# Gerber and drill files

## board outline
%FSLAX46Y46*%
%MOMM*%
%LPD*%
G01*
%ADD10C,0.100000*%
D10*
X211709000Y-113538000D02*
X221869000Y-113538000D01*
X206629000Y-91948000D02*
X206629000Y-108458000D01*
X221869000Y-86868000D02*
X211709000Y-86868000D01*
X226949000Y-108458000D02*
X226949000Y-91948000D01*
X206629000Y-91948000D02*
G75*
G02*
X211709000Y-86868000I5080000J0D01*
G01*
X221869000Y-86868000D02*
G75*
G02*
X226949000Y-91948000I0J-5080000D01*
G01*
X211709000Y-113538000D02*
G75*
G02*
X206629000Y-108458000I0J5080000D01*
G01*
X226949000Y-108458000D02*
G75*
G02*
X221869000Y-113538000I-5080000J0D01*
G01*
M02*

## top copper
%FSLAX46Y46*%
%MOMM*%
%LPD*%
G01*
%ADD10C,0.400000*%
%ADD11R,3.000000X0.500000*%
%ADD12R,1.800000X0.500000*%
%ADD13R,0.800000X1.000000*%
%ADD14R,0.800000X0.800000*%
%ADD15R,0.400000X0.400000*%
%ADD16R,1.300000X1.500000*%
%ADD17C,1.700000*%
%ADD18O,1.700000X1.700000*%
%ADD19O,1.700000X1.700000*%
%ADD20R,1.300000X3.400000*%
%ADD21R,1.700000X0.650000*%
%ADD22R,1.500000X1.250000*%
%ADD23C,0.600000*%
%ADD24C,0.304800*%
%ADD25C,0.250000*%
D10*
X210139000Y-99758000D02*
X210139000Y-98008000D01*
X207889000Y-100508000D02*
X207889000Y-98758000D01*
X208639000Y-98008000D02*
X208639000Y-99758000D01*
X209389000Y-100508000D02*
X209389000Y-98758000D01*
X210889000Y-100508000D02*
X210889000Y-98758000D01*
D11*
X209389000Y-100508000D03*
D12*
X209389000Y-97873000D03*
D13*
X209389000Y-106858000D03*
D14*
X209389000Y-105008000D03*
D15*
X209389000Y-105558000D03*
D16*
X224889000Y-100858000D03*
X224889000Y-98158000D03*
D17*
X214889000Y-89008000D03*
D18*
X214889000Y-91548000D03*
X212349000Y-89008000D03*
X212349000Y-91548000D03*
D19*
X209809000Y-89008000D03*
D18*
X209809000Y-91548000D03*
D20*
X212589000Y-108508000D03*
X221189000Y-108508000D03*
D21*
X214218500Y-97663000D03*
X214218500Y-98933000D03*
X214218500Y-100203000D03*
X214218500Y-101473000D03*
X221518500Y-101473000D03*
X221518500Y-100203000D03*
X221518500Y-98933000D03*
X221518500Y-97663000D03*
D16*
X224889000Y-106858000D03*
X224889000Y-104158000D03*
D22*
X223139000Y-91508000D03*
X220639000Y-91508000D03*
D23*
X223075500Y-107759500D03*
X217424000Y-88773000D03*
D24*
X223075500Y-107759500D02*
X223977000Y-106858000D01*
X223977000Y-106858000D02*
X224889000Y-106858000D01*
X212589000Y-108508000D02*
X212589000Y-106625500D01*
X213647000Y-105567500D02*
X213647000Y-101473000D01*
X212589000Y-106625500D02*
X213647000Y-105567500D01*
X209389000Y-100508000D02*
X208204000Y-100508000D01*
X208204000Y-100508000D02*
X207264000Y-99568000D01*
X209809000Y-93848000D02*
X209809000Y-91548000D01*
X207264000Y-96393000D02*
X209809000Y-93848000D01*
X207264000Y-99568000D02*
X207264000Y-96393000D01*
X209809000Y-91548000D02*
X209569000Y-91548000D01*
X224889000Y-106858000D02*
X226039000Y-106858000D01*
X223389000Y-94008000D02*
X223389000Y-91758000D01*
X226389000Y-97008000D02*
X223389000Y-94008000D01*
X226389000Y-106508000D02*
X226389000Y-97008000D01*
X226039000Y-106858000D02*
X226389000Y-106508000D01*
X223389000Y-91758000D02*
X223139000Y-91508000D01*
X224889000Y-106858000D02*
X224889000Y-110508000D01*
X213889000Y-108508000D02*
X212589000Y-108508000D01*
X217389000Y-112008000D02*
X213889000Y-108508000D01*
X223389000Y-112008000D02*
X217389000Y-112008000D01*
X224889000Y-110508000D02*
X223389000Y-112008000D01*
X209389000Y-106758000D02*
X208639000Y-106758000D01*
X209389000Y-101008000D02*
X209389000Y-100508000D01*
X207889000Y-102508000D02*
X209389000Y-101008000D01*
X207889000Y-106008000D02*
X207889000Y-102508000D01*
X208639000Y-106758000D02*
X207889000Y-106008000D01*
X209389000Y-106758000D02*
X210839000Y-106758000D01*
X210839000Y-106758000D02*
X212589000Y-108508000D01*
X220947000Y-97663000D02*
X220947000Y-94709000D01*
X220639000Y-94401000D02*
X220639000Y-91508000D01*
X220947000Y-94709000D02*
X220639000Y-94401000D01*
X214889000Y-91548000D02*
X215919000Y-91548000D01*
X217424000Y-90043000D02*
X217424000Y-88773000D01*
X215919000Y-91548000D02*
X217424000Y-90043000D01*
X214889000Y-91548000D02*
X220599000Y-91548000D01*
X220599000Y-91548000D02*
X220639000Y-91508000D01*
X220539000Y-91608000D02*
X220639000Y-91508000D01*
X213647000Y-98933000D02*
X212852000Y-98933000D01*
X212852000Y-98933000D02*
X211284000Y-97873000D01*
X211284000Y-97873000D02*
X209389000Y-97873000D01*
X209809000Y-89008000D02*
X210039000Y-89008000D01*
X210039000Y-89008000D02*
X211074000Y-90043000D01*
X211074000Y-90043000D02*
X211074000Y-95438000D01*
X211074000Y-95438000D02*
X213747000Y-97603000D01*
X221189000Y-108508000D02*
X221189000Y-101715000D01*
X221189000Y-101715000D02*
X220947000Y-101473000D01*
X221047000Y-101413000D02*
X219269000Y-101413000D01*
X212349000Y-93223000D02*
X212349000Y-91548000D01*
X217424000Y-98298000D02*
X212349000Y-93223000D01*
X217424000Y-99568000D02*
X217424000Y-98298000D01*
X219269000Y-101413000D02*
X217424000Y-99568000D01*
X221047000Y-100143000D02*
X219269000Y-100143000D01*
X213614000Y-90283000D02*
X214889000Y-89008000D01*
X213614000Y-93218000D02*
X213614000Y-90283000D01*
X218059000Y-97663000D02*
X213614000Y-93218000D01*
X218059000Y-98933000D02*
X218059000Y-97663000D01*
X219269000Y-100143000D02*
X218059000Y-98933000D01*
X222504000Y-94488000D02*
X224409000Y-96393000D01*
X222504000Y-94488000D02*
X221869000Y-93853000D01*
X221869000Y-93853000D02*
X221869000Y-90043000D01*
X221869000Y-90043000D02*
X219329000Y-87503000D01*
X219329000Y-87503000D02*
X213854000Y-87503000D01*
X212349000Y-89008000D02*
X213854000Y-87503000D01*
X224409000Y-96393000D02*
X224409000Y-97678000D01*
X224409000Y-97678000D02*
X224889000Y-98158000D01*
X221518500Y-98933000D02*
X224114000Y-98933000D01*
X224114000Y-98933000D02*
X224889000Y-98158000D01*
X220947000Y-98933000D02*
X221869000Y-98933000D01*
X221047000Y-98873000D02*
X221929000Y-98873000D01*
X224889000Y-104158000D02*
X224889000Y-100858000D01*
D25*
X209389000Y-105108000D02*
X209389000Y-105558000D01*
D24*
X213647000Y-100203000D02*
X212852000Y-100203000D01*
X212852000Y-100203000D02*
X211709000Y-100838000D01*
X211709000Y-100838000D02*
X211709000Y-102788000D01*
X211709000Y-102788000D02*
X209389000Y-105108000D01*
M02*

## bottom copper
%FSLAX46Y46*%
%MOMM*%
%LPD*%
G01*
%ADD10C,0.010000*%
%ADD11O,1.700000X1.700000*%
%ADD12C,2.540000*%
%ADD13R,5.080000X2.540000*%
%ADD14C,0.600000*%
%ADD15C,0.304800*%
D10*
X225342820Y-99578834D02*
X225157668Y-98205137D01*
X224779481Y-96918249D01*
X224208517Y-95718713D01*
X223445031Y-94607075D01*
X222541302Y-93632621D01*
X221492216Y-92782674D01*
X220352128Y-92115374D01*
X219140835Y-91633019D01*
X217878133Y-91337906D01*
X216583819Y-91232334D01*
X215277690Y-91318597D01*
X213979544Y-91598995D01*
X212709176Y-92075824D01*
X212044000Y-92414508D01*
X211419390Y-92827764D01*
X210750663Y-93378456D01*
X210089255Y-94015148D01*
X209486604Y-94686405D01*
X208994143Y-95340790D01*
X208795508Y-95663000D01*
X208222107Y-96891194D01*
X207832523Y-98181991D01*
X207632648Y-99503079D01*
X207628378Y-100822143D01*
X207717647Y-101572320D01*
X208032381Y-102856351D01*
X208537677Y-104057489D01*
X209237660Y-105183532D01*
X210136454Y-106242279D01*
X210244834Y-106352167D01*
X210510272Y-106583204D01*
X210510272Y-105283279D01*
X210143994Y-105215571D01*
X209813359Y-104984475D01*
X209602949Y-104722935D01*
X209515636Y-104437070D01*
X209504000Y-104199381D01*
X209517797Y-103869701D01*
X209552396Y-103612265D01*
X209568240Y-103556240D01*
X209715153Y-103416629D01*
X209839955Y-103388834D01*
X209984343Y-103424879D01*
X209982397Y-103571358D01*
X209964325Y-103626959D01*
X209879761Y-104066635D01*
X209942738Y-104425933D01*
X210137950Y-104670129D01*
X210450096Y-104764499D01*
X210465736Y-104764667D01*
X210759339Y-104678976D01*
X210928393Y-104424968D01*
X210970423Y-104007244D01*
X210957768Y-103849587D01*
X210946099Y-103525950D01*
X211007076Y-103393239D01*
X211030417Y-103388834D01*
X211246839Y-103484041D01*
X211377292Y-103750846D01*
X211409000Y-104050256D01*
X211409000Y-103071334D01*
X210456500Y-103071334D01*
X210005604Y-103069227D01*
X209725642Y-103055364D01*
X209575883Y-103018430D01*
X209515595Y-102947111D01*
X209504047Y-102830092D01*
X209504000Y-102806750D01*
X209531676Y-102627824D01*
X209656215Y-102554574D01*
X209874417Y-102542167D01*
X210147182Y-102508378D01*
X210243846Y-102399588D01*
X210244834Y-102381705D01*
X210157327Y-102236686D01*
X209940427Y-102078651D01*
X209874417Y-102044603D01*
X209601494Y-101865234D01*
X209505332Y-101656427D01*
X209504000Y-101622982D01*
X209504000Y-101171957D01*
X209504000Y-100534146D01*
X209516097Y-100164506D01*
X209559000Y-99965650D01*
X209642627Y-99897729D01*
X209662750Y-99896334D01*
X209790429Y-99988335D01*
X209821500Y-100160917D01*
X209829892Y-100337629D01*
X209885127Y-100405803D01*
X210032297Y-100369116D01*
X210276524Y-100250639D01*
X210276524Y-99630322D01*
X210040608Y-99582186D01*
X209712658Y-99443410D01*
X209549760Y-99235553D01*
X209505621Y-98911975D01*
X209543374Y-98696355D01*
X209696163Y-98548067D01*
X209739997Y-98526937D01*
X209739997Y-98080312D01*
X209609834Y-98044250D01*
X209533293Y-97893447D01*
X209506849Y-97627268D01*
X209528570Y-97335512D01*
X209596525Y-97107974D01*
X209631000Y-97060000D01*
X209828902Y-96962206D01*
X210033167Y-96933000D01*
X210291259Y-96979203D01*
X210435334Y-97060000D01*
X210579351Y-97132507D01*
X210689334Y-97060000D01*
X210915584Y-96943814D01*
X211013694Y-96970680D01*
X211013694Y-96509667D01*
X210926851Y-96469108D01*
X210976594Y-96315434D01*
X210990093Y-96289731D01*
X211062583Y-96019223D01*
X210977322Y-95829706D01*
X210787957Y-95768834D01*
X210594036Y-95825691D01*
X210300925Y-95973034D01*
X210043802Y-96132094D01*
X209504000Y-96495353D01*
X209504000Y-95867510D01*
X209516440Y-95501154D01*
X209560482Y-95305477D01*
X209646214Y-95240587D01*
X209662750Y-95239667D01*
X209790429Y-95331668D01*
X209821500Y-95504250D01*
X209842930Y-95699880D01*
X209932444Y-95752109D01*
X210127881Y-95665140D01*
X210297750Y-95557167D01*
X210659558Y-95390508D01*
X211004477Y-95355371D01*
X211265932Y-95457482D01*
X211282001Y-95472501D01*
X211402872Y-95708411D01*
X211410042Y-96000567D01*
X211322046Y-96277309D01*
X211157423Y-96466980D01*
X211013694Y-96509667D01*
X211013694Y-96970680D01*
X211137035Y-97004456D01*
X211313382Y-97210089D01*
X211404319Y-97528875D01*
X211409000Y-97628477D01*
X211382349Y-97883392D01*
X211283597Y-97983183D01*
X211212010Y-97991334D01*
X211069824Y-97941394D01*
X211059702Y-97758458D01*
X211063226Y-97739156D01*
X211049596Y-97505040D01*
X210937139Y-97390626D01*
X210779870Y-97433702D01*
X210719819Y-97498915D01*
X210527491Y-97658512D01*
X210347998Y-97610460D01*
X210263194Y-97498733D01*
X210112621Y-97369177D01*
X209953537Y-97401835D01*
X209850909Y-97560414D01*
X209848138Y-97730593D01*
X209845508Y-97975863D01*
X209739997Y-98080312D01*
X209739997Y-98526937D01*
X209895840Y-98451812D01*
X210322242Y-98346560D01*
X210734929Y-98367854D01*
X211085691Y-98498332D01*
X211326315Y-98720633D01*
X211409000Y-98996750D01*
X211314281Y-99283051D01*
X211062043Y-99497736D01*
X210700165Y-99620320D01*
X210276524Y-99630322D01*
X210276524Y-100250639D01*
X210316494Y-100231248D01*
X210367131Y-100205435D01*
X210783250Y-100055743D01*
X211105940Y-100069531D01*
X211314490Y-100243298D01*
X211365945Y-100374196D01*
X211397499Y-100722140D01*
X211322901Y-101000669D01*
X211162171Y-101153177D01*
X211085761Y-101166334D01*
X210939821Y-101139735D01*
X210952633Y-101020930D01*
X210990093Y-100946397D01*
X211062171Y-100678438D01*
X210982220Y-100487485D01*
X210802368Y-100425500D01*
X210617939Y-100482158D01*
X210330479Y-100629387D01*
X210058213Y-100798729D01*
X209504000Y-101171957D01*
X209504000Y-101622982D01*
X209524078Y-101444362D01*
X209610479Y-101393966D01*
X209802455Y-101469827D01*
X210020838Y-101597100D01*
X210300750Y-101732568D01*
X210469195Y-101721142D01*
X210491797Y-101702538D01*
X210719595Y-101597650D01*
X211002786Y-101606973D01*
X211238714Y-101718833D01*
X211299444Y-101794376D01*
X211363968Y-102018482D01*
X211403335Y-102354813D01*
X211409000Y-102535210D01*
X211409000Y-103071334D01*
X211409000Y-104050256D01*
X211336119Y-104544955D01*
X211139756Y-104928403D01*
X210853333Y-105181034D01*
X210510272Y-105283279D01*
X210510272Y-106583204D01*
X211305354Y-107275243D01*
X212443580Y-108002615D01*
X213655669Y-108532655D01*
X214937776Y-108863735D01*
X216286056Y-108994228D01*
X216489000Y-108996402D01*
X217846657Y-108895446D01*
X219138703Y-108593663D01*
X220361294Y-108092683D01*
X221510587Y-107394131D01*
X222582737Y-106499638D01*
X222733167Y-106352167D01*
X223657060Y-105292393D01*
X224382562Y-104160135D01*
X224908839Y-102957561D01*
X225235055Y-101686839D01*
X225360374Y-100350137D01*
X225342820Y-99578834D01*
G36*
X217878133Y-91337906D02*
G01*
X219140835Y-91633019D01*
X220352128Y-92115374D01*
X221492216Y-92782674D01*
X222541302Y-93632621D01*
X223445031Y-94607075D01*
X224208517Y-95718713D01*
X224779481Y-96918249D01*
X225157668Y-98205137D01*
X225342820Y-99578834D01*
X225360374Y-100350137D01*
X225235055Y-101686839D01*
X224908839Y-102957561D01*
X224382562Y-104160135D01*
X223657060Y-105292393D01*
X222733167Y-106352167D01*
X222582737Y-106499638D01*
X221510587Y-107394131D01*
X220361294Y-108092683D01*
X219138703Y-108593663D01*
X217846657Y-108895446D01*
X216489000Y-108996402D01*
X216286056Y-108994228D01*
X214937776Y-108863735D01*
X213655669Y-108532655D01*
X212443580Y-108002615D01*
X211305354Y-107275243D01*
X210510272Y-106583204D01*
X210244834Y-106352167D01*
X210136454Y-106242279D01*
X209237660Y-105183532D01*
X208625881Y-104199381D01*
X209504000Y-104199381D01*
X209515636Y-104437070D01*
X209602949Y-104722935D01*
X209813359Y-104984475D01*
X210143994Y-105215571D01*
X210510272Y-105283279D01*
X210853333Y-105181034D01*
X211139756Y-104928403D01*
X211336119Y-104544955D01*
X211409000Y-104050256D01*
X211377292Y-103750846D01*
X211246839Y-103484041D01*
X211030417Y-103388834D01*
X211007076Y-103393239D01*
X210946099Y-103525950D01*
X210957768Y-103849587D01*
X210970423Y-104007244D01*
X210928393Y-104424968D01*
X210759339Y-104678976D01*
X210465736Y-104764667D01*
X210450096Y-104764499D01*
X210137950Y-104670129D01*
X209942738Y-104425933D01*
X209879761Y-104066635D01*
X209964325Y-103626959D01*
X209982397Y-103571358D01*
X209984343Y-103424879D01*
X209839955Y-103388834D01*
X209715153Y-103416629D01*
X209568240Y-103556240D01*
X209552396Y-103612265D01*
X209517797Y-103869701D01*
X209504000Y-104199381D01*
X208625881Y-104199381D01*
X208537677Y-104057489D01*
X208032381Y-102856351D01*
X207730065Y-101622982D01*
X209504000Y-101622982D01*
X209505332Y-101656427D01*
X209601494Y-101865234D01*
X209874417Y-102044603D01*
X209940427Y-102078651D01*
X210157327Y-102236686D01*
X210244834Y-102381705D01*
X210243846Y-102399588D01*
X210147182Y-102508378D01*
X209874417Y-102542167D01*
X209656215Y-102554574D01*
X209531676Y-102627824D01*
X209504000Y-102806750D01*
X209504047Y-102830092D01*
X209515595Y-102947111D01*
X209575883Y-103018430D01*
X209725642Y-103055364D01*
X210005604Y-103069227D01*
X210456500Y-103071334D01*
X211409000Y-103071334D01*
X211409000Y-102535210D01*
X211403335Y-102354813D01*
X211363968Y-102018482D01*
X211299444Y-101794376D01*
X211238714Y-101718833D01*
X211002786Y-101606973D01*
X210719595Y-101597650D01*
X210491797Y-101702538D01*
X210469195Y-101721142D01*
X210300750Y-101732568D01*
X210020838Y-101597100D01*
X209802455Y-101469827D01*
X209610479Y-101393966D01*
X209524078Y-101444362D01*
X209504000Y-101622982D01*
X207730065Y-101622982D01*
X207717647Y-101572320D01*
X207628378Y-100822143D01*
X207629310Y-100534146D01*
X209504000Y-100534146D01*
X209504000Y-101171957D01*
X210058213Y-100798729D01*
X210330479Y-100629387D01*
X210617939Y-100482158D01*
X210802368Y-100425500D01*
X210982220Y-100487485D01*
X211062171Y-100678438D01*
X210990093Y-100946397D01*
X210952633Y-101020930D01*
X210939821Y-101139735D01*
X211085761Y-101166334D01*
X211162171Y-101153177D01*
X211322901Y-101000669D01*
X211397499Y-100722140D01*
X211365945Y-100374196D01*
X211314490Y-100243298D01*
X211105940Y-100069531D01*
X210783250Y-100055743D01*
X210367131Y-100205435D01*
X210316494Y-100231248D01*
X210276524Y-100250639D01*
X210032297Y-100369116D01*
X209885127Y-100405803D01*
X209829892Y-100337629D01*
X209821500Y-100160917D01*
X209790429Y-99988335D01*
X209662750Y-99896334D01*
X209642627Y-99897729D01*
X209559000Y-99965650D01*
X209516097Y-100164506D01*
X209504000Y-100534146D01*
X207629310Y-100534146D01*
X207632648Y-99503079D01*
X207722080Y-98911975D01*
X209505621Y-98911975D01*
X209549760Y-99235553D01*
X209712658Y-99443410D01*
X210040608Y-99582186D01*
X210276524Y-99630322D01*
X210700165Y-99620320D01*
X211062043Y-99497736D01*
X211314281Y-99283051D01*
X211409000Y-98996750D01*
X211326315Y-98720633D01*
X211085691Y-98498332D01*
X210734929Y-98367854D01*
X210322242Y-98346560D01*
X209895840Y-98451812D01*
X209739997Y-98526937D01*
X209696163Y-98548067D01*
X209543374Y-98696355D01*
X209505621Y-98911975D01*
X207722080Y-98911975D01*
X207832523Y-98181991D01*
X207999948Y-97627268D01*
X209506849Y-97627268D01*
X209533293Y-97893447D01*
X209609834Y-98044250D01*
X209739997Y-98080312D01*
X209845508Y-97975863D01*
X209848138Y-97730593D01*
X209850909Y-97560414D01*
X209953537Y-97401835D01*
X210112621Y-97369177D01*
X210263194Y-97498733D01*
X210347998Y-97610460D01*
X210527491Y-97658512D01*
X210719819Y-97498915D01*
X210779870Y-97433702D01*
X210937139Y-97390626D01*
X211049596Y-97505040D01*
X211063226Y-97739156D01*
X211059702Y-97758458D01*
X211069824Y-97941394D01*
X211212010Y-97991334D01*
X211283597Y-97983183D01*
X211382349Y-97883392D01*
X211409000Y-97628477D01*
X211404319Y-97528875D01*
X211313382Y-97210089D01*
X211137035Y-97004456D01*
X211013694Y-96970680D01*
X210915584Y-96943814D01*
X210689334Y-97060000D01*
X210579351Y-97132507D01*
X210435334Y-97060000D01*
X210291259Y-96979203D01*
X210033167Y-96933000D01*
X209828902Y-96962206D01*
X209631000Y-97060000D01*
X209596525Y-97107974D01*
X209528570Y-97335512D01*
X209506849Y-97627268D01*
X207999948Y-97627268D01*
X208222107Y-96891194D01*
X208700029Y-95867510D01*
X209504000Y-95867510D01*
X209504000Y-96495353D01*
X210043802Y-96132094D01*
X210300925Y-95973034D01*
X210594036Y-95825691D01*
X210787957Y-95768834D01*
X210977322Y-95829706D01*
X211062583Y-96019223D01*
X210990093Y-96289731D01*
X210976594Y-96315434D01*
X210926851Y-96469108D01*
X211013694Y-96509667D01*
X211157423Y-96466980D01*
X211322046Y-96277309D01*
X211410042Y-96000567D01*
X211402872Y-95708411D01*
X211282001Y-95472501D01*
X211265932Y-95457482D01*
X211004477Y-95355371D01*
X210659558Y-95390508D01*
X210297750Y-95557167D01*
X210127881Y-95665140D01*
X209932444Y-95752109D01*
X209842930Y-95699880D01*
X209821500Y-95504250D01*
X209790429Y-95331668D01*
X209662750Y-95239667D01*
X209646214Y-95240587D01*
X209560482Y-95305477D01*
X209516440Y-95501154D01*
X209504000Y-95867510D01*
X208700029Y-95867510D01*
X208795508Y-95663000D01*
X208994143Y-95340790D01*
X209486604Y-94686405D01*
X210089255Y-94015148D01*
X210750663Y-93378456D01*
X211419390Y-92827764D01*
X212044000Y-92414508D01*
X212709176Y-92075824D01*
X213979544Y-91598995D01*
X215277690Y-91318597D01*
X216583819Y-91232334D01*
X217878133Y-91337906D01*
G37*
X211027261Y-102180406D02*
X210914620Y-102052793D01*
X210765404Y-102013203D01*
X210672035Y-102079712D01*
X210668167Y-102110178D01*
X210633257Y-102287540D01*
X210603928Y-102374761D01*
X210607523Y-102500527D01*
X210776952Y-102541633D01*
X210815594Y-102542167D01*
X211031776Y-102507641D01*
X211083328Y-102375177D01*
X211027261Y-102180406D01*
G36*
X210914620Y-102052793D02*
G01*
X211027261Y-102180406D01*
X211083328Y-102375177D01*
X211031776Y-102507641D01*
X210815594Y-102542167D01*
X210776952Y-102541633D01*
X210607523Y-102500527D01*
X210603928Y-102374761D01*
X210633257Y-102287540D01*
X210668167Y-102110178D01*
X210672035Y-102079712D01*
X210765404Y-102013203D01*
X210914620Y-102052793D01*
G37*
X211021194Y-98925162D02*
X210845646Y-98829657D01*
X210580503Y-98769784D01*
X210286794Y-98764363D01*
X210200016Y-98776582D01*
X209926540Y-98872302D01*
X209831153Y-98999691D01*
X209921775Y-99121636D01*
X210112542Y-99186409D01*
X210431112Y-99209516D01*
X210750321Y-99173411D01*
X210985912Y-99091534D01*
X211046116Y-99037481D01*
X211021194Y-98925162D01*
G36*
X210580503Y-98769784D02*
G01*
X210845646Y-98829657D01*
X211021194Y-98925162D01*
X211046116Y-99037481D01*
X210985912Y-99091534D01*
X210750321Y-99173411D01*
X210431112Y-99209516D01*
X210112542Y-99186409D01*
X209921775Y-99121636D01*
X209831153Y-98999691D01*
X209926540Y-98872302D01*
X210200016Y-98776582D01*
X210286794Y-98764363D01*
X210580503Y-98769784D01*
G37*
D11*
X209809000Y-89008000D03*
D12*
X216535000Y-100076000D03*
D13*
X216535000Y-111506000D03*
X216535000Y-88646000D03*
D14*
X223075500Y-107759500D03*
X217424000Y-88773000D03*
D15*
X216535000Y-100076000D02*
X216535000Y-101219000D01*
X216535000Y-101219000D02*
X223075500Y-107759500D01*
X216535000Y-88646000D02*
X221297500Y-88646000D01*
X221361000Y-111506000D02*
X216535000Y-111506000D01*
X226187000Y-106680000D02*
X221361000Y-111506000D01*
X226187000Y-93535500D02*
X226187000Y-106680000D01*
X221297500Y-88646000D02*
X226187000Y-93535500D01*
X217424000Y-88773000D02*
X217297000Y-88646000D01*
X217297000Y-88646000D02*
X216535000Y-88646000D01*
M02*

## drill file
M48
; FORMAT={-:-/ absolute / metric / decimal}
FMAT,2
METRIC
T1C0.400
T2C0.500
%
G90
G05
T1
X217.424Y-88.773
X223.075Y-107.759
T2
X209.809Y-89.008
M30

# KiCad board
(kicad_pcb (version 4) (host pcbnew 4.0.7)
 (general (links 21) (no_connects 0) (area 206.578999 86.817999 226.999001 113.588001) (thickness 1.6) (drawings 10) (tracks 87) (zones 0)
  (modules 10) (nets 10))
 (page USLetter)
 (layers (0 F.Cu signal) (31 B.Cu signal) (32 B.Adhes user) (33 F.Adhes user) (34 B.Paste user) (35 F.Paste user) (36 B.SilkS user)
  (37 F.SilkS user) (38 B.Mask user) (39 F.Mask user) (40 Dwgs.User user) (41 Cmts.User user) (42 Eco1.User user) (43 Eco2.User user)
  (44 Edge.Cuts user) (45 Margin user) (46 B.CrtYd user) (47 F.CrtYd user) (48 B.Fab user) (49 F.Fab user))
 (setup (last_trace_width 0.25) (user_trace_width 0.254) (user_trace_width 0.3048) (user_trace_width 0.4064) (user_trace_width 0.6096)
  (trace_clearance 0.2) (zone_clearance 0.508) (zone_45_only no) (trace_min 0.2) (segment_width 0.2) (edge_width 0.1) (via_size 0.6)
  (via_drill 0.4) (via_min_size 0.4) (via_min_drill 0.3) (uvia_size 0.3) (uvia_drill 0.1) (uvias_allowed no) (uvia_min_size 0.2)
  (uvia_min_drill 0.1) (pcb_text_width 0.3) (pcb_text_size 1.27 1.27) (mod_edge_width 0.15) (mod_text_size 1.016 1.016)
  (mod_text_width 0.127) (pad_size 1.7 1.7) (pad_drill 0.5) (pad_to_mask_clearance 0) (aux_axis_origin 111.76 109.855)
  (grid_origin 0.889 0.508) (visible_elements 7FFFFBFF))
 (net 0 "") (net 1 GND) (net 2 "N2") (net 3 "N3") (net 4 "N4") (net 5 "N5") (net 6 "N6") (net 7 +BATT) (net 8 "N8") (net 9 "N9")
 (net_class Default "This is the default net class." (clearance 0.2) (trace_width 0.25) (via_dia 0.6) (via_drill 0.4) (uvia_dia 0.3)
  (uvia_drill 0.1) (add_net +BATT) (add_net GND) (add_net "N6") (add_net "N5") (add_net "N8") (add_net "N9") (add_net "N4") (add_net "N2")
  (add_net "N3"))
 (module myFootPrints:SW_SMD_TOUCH (layer F.Cu) (at 209.389 98.508 180)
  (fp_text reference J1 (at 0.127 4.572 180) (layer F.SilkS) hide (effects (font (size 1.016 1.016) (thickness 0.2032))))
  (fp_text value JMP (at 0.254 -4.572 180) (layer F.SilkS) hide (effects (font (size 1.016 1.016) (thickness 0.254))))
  (fp_line (start -0.75 -1.25) (end -0.75 0.5) (layer F.Cu) (width 0.4))
  (fp_line (start 1.5 -2) (end 1.5 -0.25) (layer F.Cu) (width 0.4))
  (fp_line (start 0.75 0.5) (end 0.75 -1.25) (layer F.Cu) (width 0.4))
  (fp_line (start 0 -2) (end 0 -0.25) (layer F.Cu) (width 0.4))
  (fp_line (start -1.5 -2) (end -1.5 -0.25) (layer F.Cu) (width 0.4))
  (pad 1 smd rect (at 0 -2 180) (size 3 0.5) (layers F.Cu F.Paste F.Mask) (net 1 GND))
  (pad 2 smd rect (at 0 0.635 180) (size 1.8 0.5) (layers F.Cu F.Paste F.Mask) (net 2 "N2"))
  (pad 3 smd circle (at 0 -0.75 180) (size 3.5 3.5) (layers F.Paste F.Mask)))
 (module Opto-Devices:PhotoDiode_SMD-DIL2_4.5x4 (layer F.Cu) (at 209.389 106.008 270)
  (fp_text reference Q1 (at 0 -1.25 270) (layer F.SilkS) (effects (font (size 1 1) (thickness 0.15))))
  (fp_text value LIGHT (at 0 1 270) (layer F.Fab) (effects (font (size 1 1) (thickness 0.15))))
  (pad 2 smd rect (at 0.85 0 90) (size 1 0.8) (layers F.Cu F.Paste F.Mask) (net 1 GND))
  (pad 1 smd rect (at -1 0 90) (size 0.8 0.8) (layers F.Cu F.Paste F.Mask) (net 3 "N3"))
  (pad 1 smd rect (at -0.45 0 90) (size 0.4 0.4) (layers F.Cu F.Paste F.Mask) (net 3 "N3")))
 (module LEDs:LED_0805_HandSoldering (layer F.Cu) (at 224.889 99.508 90)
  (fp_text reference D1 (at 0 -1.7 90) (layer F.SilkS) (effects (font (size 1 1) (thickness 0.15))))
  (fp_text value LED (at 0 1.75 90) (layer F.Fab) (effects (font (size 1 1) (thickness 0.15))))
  (pad 1 smd rect (at -1.35 0 90) (size 1.5 1.3) (layers F.Cu F.Paste F.Mask) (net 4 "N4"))
  (pad 2 smd rect (at 1.35 0 90) (size 1.5 1.3) (layers F.Cu F.Paste F.Mask) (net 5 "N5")))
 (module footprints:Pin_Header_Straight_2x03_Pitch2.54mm (layer F.Cu) (at 214.889 89.008 270)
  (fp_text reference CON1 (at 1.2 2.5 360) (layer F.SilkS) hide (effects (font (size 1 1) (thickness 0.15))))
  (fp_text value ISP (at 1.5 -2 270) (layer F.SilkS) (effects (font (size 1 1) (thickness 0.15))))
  (pad 1 smd circle (at 0 0 270) (size 1.7 1.7) (layers F.Cu F.Paste F.Mask) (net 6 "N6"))
  (pad 2 smd oval (at 2.54 0 270) (size 1.7 1.7) (layers F.Cu F.Paste F.Mask) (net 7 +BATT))
  (pad 3 smd oval (at 0 2.54 270) (size 1.7 1.7) (layers F.Cu F.Paste F.Mask) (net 5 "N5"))
  (pad 4 smd oval (at 2.54 2.54 270) (size 1.7 1.7) (layers F.Cu F.Paste F.Mask) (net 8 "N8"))
  (pad 5 thru_hole oval (at 0 5.08 270) (size 1.7 1.7) (drill 0.5) (layers *.Cu F.Mask) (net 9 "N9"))
  (pad 6 smd oval (at 2.54 5.08 270) (size 1.7 1.7) (layers F.Cu F.Paste F.Mask) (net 1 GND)))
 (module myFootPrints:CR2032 (layer B.Cu) (at 216.489 100.108 90)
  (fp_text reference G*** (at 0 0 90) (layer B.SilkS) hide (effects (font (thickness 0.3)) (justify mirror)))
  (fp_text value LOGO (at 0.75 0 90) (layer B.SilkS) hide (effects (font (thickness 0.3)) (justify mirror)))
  (fp_poly
   (pts (xy 0.529166 8.85382) (xy 1.902863 8.668668) (xy 3.189751 8.290481) (xy 4.389287 7.719517) (xy 5.500925 6.956031)
    (xy 6.475379 6.052302) (xy 7.325326 5.003216) (xy 7.992626 3.863128) (xy 8.474981 2.651835) (xy 8.770094 1.389133)
    (xy 8.875666 0.094819) (xy 8.789403 -1.21131) (xy 8.509005 -2.509456) (xy 8.032176 -3.779824) (xy 7.693492 -4.445)
    (xy 7.280236 -5.06961) (xy 6.729544 -5.738337) (xy 6.092852 -6.399745) (xy 5.421595 -7.002396) (xy 4.76721 -7.494857)
    (xy 4.445 -7.693492) (xy 3.216806 -8.266893) (xy 1.926009 -8.656477) (xy 0.604921 -8.856352) (xy -0.714143 -8.860622)
    (xy -1.46432 -8.771353) (xy -2.748351 -8.456619) (xy -3.949489 -7.951323) (xy -5.075532 -7.25134) (xy -6.134279 -6.352546)
    (xy -6.244167 -6.244166) (xy -6.475204 -5.978728) (xy -5.175279 -5.978728) (xy -5.107571 -6.345006) (xy -4.876475 -6.675641)
    (xy -4.614935 -6.886051) (xy -4.32907 -6.973364) (xy -4.091381 -6.985) (xy -3.761701 -6.971203) (xy -3.504265 -6.936604)
    (xy -3.44824 -6.92076) (xy -3.308629 -6.773847) (xy -3.280834 -6.649045) (xy -3.316879 -6.504657) (xy -3.463358 -6.506603)
    (xy -3.518959 -6.524675) (xy -3.958635 -6.609239) (xy -4.317933 -6.546262) (xy -4.562129 -6.35105) (xy -4.656499 -6.038904)
    (xy -4.656667 -6.023264) (xy -4.570976 -5.729661) (xy -4.316968 -5.560607) (xy -3.899244 -5.518577) (xy -3.741587 -5.531232)
    (xy -3.41795 -5.542901) (xy -3.285239 -5.481924) (xy -3.280834 -5.458583) (xy -3.376041 -5.242161) (xy -3.642846 -5.111708)
    (xy -3.942256 -5.08) (xy -2.963334 -5.08) (xy -2.963334 -6.0325) (xy -2.961227 -6.483396) (xy -2.947364 -6.763358)
    (xy -2.91043 -6.913117) (xy -2.839111 -6.973405) (xy -2.722092 -6.984953) (xy -2.69875 -6.985) (xy -2.519824 -6.957324)
    (xy -2.446574 -6.832785) (xy -2.434167 -6.614583) (xy -2.400378 -6.341818) (xy -2.291588 -6.245154) (xy -2.273705 -6.244166)
    (xy -2.128686 -6.331673) (xy -1.970651 -6.548573) (xy -1.936603 -6.614583) (xy -1.757234 -6.887506) (xy -1.548427 -6.983668)
    (xy -1.514982 -6.985) (xy -1.063957 -6.985) (xy -0.426146 -6.985) (xy -0.056506 -6.972903) (xy 0.14235 -6.93) (xy 0.210271 -6.846373)
    (xy 0.211666 -6.82625) (xy 0.119665 -6.698571) (xy -0.052917 -6.6675) (xy -0.229629 -6.659108) (xy -0.297803 -6.603873)
    (xy -0.261116 -6.456703) (xy -0.142639 -6.212476) (xy 0.477678 -6.212476) (xy 0.525814 -6.448392) (xy 0.66459 -6.776342)
    (xy 0.872447 -6.93924) (xy 1.196025 -6.983379) (xy 1.411645 -6.945626) (xy 1.559933 -6.792837) (xy 1.581063 -6.749003)
    (xy 2.027688 -6.749003) (xy 2.06375 -6.879166) (xy 2.214553 -6.955707) (xy 2.480732 -6.982151) (xy 2.772488 -6.96043)
    (xy 3.000026 -6.892475) (xy 3.048 -6.858) (xy 3.145794 -6.660098) (xy 3.175 -6.455833) (xy 3.128797 -6.197741) (xy 3.048 -6.053666)
    (xy 2.975493 -5.909649) (xy 3.048 -5.799666) (xy 3.164186 -5.573416) (xy 3.13732 -5.475306) (xy 3.598333 -5.475306)
    (xy 3.638892 -5.562149) (xy 3.792566 -5.512406) (xy 3.818269 -5.498907) (xy 4.088777 -5.426417) (xy 4.278294 -5.511678)
    (xy 4.339166 -5.701043) (xy 4.282309 -5.894964) (xy 4.134966 -6.188075) (xy 3.975906 -6.445198) (xy 3.612647 -6.985) (xy 4.24049 -6.985)
    (xy 4.606846 -6.97256) (xy 4.802523 -6.928518) (xy 4.867413 -6.842786) (xy 4.868333 -6.82625) (xy 4.776332 -6.698571)
    (xy 4.60375 -6.6675) (xy 4.40812 -6.64607) (xy 4.355891 -6.556556) (xy 4.44286 -6.361119) (xy 4.550833 -6.19125) (xy 4.717492 -5.829442)
    (xy 4.752629 -5.484523) (xy 4.650518 -5.223068) (xy 4.635499 -5.206999) (xy 4.399589 -5.086128) (xy 4.107433 -5.078958)
    (xy 3.830691 -5.166954) (xy 3.64102 -5.331577) (xy 3.598333 -5.475306) (xy 3.13732 -5.475306) (xy 3.103544 -5.351965)
    (xy 2.897911 -5.175618) (xy 2.579125 -5.084681) (xy 2.479523 -5.08) (xy 2.224608 -5.106651) (xy 2.124817 -5.205403)
    (xy 2.116666 -5.27699) (xy 2.166606 -5.419176) (xy 2.349542 -5.429298) (xy 2.368844 -5.425774) (xy 2.60296 -5.439404)
    (xy 2.717374 -5.551861) (xy 2.674298 -5.70913) (xy 2.609085 -5.769181) (xy 2.449488 -5.961509) (xy 2.49754 -6.141002)
    (xy 2.609267 -6.225806) (xy 2.738823 -6.376379) (xy 2.706165 -6.535463) (xy 2.547586 -6.638091) (xy 2.377407 -6.640862)
    (xy 2.132137 -6.643492) (xy 2.027688 -6.749003) (xy 1.581063 -6.749003) (xy 1.656188 -6.59316) (xy 1.76144 -6.166758)
    (xy 1.740146 -5.754071) (xy 1.609668 -5.403309) (xy 1.387367 -5.162685) (xy 1.11125 -5.08) (xy 0.824949 -5.174719)
    (xy 0.610264 -5.426957) (xy 0.48768 -5.788835) (xy 0.477678 -6.212476) (xy -0.142639 -6.212476) (xy -0.123248 -6.172506)
    (xy -0.097435 -6.121869) (xy 0.052257 -5.70575) (xy 0.038469 -5.38306) (xy -0.135298 -5.17451) (xy -0.266196 -5.123055)
    (xy -0.61414 -5.091501) (xy -0.892669 -5.166099) (xy -1.045177 -5.326829) (xy -1.058334 -5.403239) (xy -1.031735 -5.549179)
    (xy -0.91293 -5.536367) (xy -0.838397 -5.498907) (xy -0.570438 -5.426829) (xy -0.379485 -5.50678) (xy -0.3175 -5.686632)
    (xy -0.374158 -5.871061) (xy -0.521387 -6.158521) (xy -0.690729 -6.430787) (xy -1.063957 -6.985) (xy -1.514982 -6.985)
    (xy -1.336362 -6.964922) (xy -1.285966 -6.878521) (xy -1.361827 -6.686545) (xy -1.4891 -6.468162) (xy -1.624568 -6.18825)
    (xy -1.613142 -6.019805) (xy -1.594538 -5.997203) (xy -1.48965 -5.769405) (xy -1.498973 -5.486214) (xy -1.610833 -5.250286)
    (xy -1.686376 -5.189556) (xy -1.910482 -5.125032) (xy -2.246813 -5.085665) (xy -2.42721 -5.08) (xy -2.963334 -5.08) (xy -3.942256 -5.08)
    (xy -4.436955 -5.152881) (xy -4.820403 -5.349244) (xy -5.073034 -5.635667) (xy -5.175279 -5.978728) (xy -6.475204 -5.978728)
    (xy -7.167243 -5.183646) (xy -7.894615 -4.04542) (xy -8.424655 -2.833331) (xy -8.755735 -1.551224) (xy -8.886228 -0.202944)
    (xy -8.888402 0) (xy -8.787446 1.357657) (xy -8.485663 2.649703) (xy -7.984683 3.872294) (xy -7.286131 5.021587) (xy -6.391638 6.093737)
    (xy -6.244167 6.244167) (xy -5.184393 7.16806) (xy -4.052135 7.893562) (xy -2.849561 8.419839) (xy -1.578839 8.746055)
    (xy -0.242137 8.871374) (xy 0.529166 8.85382))
   (layer B.Cu) (width 0.01))
  (fp_poly
   (pts (xy -2.072406 -5.461739) (xy -1.944793 -5.57438) (xy -1.905203 -5.723596) (xy -1.971712 -5.816965) (xy -2.002178 -5.820833)
    (xy -2.17954 -5.855743) (xy -2.266761 -5.885072) (xy -2.392527 -5.881477) (xy -2.433633 -5.712048) (xy -2.434167 -5.673406)
    (xy -2.399641 -5.457224) (xy -2.267177 -5.405672) (xy -2.072406 -5.461739))
   (layer B.Cu) (width 0.01))
  (fp_poly
   (pts (xy 1.182838 -5.467806) (xy 1.278343 -5.643354) (xy 1.338216 -5.908497) (xy 1.343637 -6.202206) (xy 1.331418 -6.288984)
    (xy 1.235698 -6.56246) (xy 1.108309 -6.657847) (xy 0.986364 -6.567225) (xy 0.921591 -6.376458) (xy 0.898484 -6.057888)
    (xy 0.934589 -5.738679) (xy 1.016466 -5.503088) (xy 1.070519 -5.442884) (xy 1.182838 -5.467806))
   (layer B.Cu) (width 0.01))
  (pad 3 smd circle (at 0 0 90) (size 17.78 17.78) (layers B.Paste B.Mask)))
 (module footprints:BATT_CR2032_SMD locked (layer B.Cu) (at 216.535 100.076 90)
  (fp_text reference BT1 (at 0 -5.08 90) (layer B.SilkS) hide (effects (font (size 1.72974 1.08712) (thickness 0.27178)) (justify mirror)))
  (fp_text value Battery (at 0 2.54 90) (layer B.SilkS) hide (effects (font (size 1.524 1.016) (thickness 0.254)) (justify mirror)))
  (pad 2 smd circle (at 0 0 90) (size 2.54 2.54) (layers B.Cu B.Paste B.Mask) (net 1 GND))
  (pad 1 smd rect (at -11.43 0 90) (size 2.54 5.08) (layers B.Cu B.Paste B.Mask) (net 7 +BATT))
  (pad 1 smd rect (at 11.43 0 90) (size 2.54 5.08) (layers B.Cu B.Paste B.Mask) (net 7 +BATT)))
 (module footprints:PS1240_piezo (layer F.Cu) (at 216.889 108.508)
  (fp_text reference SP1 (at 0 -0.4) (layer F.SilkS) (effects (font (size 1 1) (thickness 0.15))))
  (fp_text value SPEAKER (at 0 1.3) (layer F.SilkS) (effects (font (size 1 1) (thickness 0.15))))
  (pad 1 smd rect (at -4.3 0) (size 1.3 3.4) (layers F.Cu F.Paste F.Mask) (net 1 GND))
  (pad 2 smd rect (at 4.3 0) (size 1.3 3.4) (layers F.Cu F.Paste F.Mask) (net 8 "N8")))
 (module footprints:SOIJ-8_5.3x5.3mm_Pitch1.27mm (layer F.Cu) (at 217.8685 99.568)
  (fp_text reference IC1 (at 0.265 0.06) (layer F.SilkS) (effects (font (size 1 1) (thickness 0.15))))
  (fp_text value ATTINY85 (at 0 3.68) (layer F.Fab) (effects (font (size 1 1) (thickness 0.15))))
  (pad 1 smd rect (at -3.65 -1.905) (size 1.7 0.65) (layers F.Cu F.Paste F.Mask) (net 9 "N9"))
  (pad 2 smd rect (at -3.65 -0.635) (size 1.7 0.65) (layers F.Cu F.Paste F.Mask) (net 2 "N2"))
  (pad 3 smd rect (at -3.65 0.635) (size 1.7 0.65) (layers F.Cu F.Paste F.Mask) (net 3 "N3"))
  (pad 4 smd rect (at -3.65 1.905) (size 1.7 0.65) (layers F.Cu F.Paste F.Mask) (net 1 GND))
  (pad 5 smd rect (at 3.65 1.905) (size 1.7 0.65) (layers F.Cu F.Paste F.Mask) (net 8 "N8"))
  (pad 6 smd rect (at 3.65 0.635) (size 1.7 0.65) (layers F.Cu F.Paste F.Mask) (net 6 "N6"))
  (pad 7 smd rect (at 3.65 -0.635) (size 1.7 0.65) (layers F.Cu F.Paste F.Mask) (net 5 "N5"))
  (pad 8 smd rect (at 3.65 -1.905) (size 1.7 0.65) (layers F.Cu F.Paste F.Mask) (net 7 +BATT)))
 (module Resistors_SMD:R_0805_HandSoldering (layer F.Cu) (at 224.889 105.508 90)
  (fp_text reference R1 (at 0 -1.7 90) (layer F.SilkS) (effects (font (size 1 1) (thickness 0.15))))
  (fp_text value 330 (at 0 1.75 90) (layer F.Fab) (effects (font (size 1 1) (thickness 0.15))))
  (pad 1 smd rect (at -1.35 0 90) (size 1.5 1.3) (layers F.Cu F.Paste F.Mask) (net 1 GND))
  (pad 2 smd rect (at 1.35 0 90) (size 1.5 1.3) (layers F.Cu F.Paste F.Mask) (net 4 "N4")))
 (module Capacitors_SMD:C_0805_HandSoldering (layer F.Cu) (at 221.889 91.508 180)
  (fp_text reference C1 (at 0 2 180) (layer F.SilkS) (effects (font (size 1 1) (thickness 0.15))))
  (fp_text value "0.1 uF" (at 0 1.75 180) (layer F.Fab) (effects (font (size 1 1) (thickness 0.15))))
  (pad 1 smd rect (at -1.25 0 180) (size 1.5 1.25) (layers F.Cu F.Paste F.Mask) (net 1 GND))
  (pad 2 smd rect (at 1.25 0 180) (size 1.5 1.25) (layers F.Cu F.Paste F.Mask) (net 7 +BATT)))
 (gr_line (start 211.709 113.538) (end 221.869 113.538) (angle 90) (layer Edge.Cuts) (width 0.1))
 (gr_line (start 206.629 91.948) (end 206.629 108.458) (angle 90) (layer Edge.Cuts) (width 0.1))
 (gr_line (start 221.869 86.868) (end 211.709 86.868) (angle 90) (layer Edge.Cuts) (width 0.1))
 (gr_line (start 226.949 108.458) (end 226.949 91.948) (angle 90) (layer Edge.Cuts) (width 0.1))
 (gr_arc (start 211.709 91.948) (end 206.629 91.948) (angle 90) (layer Edge.Cuts) (width 0.1))
 (gr_arc (start 221.869 91.948) (end 221.869 86.868) (angle 90) (layer Edge.Cuts) (width 0.1))
 (gr_arc (start 211.709 108.458) (end 211.709 113.538) (angle 90) (layer Edge.Cuts) (width 0.1))
 (gr_arc (start 221.869 108.458) (end 226.949 108.458) (angle 90) (layer Edge.Cuts) (width 0.1))
 (segment (start 216.535 100.076) (end 216.535 101.219) (width 0.3048) (layer B.Cu) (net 1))
 (segment (start 216.535 101.219) (end 223.0755 107.7595) (width 0.3048) (layer B.Cu) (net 1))
 (via (at 223.0755 107.7595) (size 0.6) (drill 0.4) (layers F.Cu B.Cu) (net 1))
 (segment (start 223.0755 107.7595) (end 223.977 106.858) (width 0.3048) (layer F.Cu) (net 1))
 (segment (start 223.977 106.858) (end 224.889 106.858) (width 0.3048) (layer F.Cu) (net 1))
 (segment (start 212.589 108.508) (end 212.589 106.6255) (width 0.3048) (layer F.Cu) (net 1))
 (segment (start 213.647 105.5675) (end 213.647 101.473) (width 0.3048) (layer F.Cu) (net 1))
 (segment (start 212.589 106.6255) (end 213.647 105.5675) (width 0.3048) (layer F.Cu) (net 1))
 (segment (start 209.389 100.508) (end 208.204 100.508) (width 0.3048) (layer F.Cu) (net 1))
 (segment (start 208.204 100.508) (end 207.264 99.568) (width 0.3048) (layer F.Cu) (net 1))
 (segment (start 209.809 93.848) (end 209.809 91.548) (width 0.3048) (layer F.Cu) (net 1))
 (segment (start 207.264 96.393) (end 209.809 93.848) (width 0.3048) (layer F.Cu) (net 1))
 (segment (start 207.264 99.568) (end 207.264 96.393) (width 0.3048) (layer F.Cu) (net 1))
 (segment (start 209.809 91.548) (end 209.569 91.548) (width 0.3048) (layer F.Cu) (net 1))
 (segment (start 224.889 106.858) (end 226.039 106.858) (width 0.3048) (layer F.Cu) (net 1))
 (segment (start 223.389 94.008) (end 223.389 91.758) (width 0.3048) (layer F.Cu) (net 1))
 (segment (start 226.389 97.008) (end 223.389 94.008) (width 0.3048) (layer F.Cu) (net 1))
 (segment (start 226.389 106.508) (end 226.389 97.008) (width 0.3048) (layer F.Cu) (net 1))
 (segment (start 226.039 106.858) (end 226.389 106.508) (width 0.3048) (layer F.Cu) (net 1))
 (segment (start 223.389 91.758) (end 223.139 91.508) (width 0.3048) (layer F.Cu) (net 1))
 (segment (start 224.889 106.858) (end 224.889 110.508) (width 0.3048) (layer F.Cu) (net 1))
 (segment (start 213.889 108.508) (end 212.589 108.508) (width 0.3048) (layer F.Cu) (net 1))
 (segment (start 217.389 112.008) (end 213.889 108.508) (width 0.3048) (layer F.Cu) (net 1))
 (segment (start 223.389 112.008) (end 217.389 112.008) (width 0.3048) (layer F.Cu) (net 1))
 (segment (start 224.889 110.508) (end 223.389 112.008) (width 0.3048) (layer F.Cu) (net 1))
 (segment (start 209.389 106.758) (end 208.639 106.758) (width 0.3048) (layer F.Cu) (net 1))
 (segment (start 209.389 101.008) (end 209.389 100.508) (width 0.3048) (layer F.Cu) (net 1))
 (segment (start 207.889 102.508) (end 209.389 101.008) (width 0.3048) (layer F.Cu) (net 1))
 (segment (start 207.889 106.008) (end 207.889 102.508) (width 0.3048) (layer F.Cu) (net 1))
 (segment (start 208.639 106.758) (end 207.889 106.008) (width 0.3048) (layer F.Cu) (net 1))
 (segment (start 209.389 106.758) (end 210.839 106.758) (width 0.3048) (layer F.Cu) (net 1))
 (segment (start 210.839 106.758) (end 212.589 108.508) (width 0.3048) (layer F.Cu) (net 1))
 (segment (start 216.535 88.646) (end 221.2975 88.646) (width 0.3048) (layer B.Cu) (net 7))
 (segment (start 221.361 111.506) (end 216.535 111.506) (width 0.3048) (layer B.Cu) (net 7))
 (segment (start 226.187 106.68) (end 221.361 111.506) (width 0.3048) (layer B.Cu) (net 7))
 (segment (start 226.187 93.5355) (end 226.187 106.68) (width 0.3048) (layer B.Cu) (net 7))
 (segment (start 221.2975 88.646) (end 226.187 93.5355) (width 0.3048) (layer B.Cu) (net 7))
 (segment (start 220.947 97.663) (end 220.947 94.709) (width 0.3048) (layer F.Cu) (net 7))
 (segment (start 220.639 94.401) (end 220.639 91.508) (width 0.3048) (layer F.Cu) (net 7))
 (segment (start 220.947 94.709) (end 220.639 94.401) (width 0.3048) (layer F.Cu) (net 7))
 (segment (start 214.889 91.548) (end 215.919 91.548) (width 0.3048) (layer F.Cu) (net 7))
 (segment (start 217.424 88.773) (end 217.297 88.646) (width 0.3048) (layer B.Cu) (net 7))
 (via (at 217.424 88.773) (size 0.6) (drill 0.4) (layers F.Cu B.Cu) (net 7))
 (segment (start 217.424 90.043) (end 217.424 88.773) (width 0.3048) (layer F.Cu) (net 7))
 (segment (start 215.919 91.548) (end 217.424 90.043) (width 0.3048) (layer F.Cu) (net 7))
 (segment (start 217.297 88.646) (end 216.535 88.646) (width 0.3048) (layer B.Cu) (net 7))
 (segment (start 214.889 91.548) (end 220.599 91.548) (width 0.3048) (layer F.Cu) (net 7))
 (segment (start 220.599 91.548) (end 220.639 91.508) (width 0.3048) (layer F.Cu) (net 7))
 (segment (start 220.539 91.608) (end 220.639 91.508) (width 0.3048) (layer F.Cu) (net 7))
 (segment (start 213.647 98.933) (end 212.852 98.933) (width 0.3048) (layer F.Cu) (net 2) (status 30))
 (segment (start 212.852 98.933) (end 211.284 97.873) (width 0.3048) (layer F.Cu) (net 2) (status 10))
 (segment (start 211.284 97.873) (end 209.389 97.873) (width 0.3048) (layer F.Cu) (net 2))
 (segment (start 209.809 89.008) (end 210.039 89.008) (width 0.3048) (layer F.Cu) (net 9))
 (segment (start 210.039 89.008) (end 211.074 90.043) (width 0.3048) (layer F.Cu) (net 9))
 (segment (start 211.074 90.043) (end 211.074 95.438) (width 0.3048) (layer F.Cu) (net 9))
 (segment (start 211.074 95.438) (end 213.747 97.603) (width 0.3048) (layer F.Cu) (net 9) (status 20))
 (segment (start 221.189 108.508) (end 221.189 101.715) (width 0.3048) (layer F.Cu) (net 8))
 (segment (start 221.189 101.715) (end 220.947 101.473) (width 0.3048) (layer F.Cu) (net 8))
 (segment (start 221.047 101.413) (end 219.269 101.413) (width 0.3048) (layer F.Cu) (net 8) (status 10))
 (segment (start 212.349 93.223) (end 212.349 91.548) (width 0.3048) (layer F.Cu) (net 8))
 (segment (start 217.424 98.298) (end 212.349 93.223) (width 0.3048) (layer F.Cu) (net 8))
 (segment (start 217.424 99.568) (end 217.424 98.298) (width 0.3048) (layer F.Cu) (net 8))
 (segment (start 219.269 101.413) (end 217.424 99.568) (width 0.3048) (layer F.Cu) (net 8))
 (segment (start 221.047 100.143) (end 219.269 100.143) (width 0.3048) (layer F.Cu) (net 6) (status 10))
 (segment (start 213.614 90.283) (end 214.889 89.008) (width 0.3048) (layer F.Cu) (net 6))
 (segment (start 213.614 93.218) (end 213.614 90.283) (width 0.3048) (layer F.Cu) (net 6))
 (segment (start 218.059 97.663) (end 213.614 93.218) (width 0.3048) (layer F.Cu) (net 6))
 (segment (start 218.059 98.933) (end 218.059 97.663) (width 0.3048) (layer F.Cu) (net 6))
 (segment (start 219.269 100.143) (end 218.059 98.933) (width 0.3048) (layer F.Cu) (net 6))
 (segment (start 222.504 94.488) (end 224.409 96.393) (width 0.3048) (layer F.Cu) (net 5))
 (segment (start 222.504 94.488) (end 221.869 93.853) (width 0.3048) (layer F.Cu) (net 5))
 (segment (start 221.869 93.853) (end 221.869 90.043) (width 0.3048) (layer F.Cu) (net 5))
 (segment (start 221.869 90.043) (end 219.329 87.503) (width 0.3048) (layer F.Cu) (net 5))
 (segment (start 219.329 87.503) (end 213.854 87.503) (width 0.3048) (layer F.Cu) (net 5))
 (segment (start 212.349 89.008) (end 213.854 87.503) (width 0.3048) (layer F.Cu) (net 5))
 (segment (start 224.409 96.393) (end 224.409 97.678) (width 0.3048) (layer F.Cu) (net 5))
 (segment (start 224.409 97.678) (end 224.889 98.158) (width 0.3048) (layer F.Cu) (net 5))
 (segment (start 221.5185 98.933) (end 224.114 98.933) (width 0.3048) (layer F.Cu) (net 5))
 (segment (start 224.114 98.933) (end 224.889 98.158) (width 0.3048) (layer F.Cu) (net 5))
 (segment (start 220.947 98.933) (end 221.869 98.933) (width 0.3048) (layer F.Cu) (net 5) (status 10))
 (segment (start 221.047 98.873) (end 221.929 98.873) (width 0.3048) (layer F.Cu) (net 5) (status 10))
 (segment (start 224.889 104.158) (end 224.889 100.858) (width 0.3048) (layer F.Cu) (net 4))
 (segment (start 209.389 105.108) (end 209.389 105.558) (width 0.25) (layer F.Cu) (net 3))
 (segment (start 213.647 100.203) (end 212.852 100.203) (width 0.3048) (layer F.Cu) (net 3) (status 30))
 (segment (start 212.852 100.203) (end 211.709 100.838) (width 0.3048) (layer F.Cu) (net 3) (status 10))
 (segment (start 211.709 100.838) (end 211.709 102.788) (width 0.3048) (layer F.Cu) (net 3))
 (segment (start 211.709 102.788) (end 209.389 105.108) (width 0.3048) (layer F.Cu) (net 3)))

